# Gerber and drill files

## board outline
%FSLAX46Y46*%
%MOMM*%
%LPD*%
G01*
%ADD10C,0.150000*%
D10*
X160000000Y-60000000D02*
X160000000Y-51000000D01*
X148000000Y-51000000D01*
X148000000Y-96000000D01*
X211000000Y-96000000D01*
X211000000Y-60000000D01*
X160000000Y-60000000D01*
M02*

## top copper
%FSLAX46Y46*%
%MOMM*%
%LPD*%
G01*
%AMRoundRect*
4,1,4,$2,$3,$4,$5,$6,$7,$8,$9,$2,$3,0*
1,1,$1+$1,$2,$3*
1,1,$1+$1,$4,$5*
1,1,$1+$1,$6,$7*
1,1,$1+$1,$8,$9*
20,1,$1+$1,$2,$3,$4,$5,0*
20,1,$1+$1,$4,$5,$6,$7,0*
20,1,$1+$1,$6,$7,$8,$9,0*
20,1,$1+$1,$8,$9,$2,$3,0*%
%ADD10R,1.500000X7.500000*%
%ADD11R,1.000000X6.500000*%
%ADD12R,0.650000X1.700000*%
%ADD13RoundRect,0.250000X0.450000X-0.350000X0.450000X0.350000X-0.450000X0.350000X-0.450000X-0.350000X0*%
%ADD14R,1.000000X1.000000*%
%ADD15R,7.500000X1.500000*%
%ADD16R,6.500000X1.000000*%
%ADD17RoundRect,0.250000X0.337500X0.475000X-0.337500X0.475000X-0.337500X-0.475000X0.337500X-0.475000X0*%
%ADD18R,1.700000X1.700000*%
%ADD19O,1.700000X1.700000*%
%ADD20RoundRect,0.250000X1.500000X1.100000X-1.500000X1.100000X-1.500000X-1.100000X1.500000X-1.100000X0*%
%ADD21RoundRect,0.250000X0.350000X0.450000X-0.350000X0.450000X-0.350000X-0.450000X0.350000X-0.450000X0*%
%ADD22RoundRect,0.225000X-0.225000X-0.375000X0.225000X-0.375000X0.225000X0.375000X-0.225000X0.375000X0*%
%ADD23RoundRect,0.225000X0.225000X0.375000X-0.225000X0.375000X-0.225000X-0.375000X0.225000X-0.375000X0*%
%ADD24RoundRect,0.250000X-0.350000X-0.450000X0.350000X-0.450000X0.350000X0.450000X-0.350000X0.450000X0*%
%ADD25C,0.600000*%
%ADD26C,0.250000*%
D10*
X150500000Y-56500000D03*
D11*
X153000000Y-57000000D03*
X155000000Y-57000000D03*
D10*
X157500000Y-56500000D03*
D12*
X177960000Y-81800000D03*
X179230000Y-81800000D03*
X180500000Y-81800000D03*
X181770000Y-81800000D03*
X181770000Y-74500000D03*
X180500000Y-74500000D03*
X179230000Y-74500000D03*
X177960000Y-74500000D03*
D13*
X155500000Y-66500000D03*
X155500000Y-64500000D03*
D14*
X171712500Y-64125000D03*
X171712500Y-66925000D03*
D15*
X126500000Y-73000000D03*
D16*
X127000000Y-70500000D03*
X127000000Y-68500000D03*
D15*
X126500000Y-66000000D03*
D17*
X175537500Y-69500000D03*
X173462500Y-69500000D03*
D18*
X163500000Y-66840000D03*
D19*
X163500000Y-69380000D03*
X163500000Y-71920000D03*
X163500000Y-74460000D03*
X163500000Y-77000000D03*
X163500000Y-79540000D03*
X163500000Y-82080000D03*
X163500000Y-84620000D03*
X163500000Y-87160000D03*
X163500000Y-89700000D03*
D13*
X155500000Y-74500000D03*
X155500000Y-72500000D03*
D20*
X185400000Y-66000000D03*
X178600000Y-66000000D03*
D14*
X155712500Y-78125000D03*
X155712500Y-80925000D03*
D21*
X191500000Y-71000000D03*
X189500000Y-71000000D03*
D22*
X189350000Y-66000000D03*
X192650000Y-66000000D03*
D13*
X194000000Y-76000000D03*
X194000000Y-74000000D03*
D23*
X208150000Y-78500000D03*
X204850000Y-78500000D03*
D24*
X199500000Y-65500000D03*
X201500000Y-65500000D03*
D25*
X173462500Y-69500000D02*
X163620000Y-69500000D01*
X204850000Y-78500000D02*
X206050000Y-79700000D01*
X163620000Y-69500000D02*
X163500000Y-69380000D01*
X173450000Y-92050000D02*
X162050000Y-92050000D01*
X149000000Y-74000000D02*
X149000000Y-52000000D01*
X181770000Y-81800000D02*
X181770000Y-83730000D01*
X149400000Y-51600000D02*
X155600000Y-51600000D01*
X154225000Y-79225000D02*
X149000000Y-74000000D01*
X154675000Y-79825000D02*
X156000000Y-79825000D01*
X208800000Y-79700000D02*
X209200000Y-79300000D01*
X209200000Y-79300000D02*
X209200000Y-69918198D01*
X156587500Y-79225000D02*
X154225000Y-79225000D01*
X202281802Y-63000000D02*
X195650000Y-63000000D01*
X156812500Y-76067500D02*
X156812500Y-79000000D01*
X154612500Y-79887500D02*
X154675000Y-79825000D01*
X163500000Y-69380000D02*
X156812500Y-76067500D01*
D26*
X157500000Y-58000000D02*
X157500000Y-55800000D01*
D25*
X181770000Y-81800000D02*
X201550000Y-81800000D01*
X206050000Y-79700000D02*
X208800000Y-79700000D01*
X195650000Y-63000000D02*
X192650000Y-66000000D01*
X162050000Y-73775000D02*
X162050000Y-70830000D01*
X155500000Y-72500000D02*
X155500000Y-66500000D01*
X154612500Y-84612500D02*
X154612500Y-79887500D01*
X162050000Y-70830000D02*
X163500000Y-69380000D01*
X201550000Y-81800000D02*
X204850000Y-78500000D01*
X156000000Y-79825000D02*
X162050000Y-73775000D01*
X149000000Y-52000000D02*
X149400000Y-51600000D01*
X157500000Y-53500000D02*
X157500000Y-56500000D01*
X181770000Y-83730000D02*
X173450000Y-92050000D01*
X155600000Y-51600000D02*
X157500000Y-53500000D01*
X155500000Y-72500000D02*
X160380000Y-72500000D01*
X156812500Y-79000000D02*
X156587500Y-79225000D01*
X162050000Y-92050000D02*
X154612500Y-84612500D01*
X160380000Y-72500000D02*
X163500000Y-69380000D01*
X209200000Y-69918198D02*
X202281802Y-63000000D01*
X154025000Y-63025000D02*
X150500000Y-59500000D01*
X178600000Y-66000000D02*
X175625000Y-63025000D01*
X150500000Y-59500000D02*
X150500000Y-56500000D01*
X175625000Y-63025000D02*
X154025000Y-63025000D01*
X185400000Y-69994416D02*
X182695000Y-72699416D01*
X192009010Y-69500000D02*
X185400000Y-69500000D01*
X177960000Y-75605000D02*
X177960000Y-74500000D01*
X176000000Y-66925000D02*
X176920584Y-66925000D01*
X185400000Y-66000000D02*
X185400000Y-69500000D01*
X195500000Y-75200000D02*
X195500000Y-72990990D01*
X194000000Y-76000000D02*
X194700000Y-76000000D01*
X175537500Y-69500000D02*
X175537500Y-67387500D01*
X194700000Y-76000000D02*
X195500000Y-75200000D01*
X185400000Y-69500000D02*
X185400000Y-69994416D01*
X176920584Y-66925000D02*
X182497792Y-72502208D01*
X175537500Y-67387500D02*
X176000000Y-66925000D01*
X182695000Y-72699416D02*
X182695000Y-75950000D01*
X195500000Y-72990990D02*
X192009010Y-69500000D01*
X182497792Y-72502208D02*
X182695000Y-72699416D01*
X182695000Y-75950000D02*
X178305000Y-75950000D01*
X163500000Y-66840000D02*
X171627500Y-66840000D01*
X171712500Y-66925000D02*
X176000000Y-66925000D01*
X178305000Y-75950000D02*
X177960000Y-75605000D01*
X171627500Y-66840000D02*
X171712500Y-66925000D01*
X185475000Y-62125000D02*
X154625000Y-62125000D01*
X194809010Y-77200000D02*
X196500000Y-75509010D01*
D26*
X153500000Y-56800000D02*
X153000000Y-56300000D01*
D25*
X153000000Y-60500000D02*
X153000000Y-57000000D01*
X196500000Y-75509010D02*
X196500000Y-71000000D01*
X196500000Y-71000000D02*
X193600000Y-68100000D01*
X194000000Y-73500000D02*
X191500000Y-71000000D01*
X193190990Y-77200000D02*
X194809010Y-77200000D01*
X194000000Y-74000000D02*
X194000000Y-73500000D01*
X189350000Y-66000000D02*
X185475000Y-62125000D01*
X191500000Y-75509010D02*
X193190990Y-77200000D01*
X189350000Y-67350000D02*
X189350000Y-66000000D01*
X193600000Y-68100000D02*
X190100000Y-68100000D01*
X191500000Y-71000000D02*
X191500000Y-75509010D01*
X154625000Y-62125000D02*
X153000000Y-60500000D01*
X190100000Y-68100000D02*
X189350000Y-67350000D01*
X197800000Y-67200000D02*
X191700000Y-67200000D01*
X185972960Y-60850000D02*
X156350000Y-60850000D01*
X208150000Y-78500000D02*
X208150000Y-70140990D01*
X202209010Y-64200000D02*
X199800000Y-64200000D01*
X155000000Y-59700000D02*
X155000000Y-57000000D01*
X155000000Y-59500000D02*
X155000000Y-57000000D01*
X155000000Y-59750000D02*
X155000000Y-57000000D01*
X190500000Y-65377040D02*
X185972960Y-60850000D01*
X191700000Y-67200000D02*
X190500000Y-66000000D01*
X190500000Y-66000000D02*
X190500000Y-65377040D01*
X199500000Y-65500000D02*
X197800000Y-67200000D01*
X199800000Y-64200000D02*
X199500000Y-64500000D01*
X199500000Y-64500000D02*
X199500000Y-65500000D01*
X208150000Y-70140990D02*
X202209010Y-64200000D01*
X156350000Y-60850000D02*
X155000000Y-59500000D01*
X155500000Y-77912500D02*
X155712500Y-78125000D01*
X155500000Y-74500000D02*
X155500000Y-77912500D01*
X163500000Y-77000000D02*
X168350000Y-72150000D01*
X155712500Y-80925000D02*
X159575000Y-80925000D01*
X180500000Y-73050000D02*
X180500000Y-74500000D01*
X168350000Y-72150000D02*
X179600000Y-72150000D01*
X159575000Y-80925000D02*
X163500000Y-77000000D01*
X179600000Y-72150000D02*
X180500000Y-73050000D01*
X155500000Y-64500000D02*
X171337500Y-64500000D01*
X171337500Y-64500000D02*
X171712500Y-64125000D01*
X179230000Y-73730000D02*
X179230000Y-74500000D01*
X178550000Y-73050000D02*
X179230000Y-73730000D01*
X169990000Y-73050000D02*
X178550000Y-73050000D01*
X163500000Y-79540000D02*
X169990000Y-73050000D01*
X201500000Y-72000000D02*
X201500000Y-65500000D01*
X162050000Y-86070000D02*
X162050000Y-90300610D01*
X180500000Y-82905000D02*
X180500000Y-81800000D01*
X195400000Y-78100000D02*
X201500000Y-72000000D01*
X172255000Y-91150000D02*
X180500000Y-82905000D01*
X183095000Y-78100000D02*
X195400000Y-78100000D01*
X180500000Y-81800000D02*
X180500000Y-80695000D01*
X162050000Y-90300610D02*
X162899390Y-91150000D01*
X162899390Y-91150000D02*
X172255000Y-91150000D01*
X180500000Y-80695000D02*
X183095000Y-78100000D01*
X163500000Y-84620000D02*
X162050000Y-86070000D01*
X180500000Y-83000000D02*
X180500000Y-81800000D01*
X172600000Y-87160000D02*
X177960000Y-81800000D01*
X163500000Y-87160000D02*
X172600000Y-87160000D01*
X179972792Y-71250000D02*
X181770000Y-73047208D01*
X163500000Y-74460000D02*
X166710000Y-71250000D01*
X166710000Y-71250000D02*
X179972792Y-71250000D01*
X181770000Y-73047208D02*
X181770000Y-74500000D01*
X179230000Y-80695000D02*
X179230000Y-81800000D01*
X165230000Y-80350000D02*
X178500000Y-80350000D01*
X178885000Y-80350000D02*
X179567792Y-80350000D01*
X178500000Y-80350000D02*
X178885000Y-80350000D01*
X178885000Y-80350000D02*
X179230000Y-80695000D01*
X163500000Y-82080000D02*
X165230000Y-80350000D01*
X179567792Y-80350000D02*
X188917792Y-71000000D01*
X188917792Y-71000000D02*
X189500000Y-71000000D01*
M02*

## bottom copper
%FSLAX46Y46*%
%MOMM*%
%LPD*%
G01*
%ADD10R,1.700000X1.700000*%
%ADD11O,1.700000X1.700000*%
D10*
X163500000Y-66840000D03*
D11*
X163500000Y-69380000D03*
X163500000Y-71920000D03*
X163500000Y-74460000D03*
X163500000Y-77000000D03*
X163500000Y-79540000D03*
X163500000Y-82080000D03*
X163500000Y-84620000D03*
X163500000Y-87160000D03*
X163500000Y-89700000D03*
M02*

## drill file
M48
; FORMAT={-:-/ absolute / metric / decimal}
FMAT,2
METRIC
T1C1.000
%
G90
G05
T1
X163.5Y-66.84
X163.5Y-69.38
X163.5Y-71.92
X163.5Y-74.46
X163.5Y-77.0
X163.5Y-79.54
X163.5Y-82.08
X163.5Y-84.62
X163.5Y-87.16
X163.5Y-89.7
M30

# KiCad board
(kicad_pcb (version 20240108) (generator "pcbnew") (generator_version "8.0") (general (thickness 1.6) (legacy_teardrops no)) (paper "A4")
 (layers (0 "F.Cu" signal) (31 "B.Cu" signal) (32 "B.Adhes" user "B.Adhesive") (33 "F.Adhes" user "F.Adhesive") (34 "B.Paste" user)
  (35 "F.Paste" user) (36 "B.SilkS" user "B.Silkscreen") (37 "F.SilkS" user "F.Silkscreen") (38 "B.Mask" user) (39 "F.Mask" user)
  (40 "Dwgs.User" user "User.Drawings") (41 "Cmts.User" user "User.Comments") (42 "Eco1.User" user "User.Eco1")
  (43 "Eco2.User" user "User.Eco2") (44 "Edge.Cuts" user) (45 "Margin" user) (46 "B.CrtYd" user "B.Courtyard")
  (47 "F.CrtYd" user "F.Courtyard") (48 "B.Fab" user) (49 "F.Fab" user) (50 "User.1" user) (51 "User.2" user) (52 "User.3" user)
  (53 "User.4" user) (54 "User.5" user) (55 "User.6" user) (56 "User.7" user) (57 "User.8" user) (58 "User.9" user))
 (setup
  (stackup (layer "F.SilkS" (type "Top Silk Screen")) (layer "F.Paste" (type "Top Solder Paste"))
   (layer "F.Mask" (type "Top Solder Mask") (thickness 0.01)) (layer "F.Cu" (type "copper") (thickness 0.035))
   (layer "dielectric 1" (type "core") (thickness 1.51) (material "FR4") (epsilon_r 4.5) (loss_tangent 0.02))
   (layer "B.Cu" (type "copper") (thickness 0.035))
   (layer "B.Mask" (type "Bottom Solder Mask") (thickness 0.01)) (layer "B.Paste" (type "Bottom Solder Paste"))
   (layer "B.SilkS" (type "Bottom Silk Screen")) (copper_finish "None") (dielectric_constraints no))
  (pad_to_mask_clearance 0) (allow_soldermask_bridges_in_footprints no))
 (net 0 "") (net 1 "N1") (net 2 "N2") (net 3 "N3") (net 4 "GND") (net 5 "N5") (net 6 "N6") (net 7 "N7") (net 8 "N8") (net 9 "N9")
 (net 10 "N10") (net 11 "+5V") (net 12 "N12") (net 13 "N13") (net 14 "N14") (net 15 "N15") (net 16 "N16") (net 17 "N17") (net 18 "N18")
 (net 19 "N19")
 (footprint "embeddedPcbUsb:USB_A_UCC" (layer "F.Cu") (at 154 56.7 -90)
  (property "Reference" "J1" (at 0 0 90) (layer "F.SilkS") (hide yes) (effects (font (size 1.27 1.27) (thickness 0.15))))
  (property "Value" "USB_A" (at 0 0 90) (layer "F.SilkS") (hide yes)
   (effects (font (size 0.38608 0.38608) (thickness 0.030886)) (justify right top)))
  (pad "1" smd rect (at -0.2 3.5 270) (size 7.5 1.5) (layers "F.Cu" "F.Paste" "F.Mask") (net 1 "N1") (solder_mask_margin 0.1016))
  (pad "2" smd rect (at 0.3 1 270) (size 6.5 1) (layers "F.Cu" "F.Paste" "F.Mask") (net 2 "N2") (solder_mask_margin 0.1016))
  (pad "3" smd rect (at 0.3 -1 270) (size 6.5 1) (layers "F.Cu" "F.Paste" "F.Mask") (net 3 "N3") (solder_mask_margin 0.1016))
  (pad "4" smd rect (at -0.2 -3.5 270) (size 7.5 1.5) (layers "F.Cu" "F.Paste" "F.Mask") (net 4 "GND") (solder_mask_margin 0.1016)))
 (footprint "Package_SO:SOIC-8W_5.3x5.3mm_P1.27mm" (layer "F.Cu") (at 179.865 78.15 90)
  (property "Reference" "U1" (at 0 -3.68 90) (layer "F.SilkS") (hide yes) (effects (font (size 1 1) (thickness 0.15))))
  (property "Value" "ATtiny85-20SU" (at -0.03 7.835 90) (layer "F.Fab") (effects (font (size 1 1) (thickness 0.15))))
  (pad "1" smd rect (at -3.65 -1.905 90) (size 1.7 0.65) (layers "F.Cu" "F.Paste" "F.Mask") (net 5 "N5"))
  (pad "2" smd rect (at -3.65 -0.635 90) (size 1.7 0.65) (layers "F.Cu" "F.Paste" "F.Mask") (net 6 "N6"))
  (pad "3" smd rect (at -3.65 0.635 90) (size 1.7 0.65) (layers "F.Cu" "F.Paste" "F.Mask") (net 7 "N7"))
  (pad "4" smd rect (at -3.65 1.905 90) (size 1.7 0.65) (layers "F.Cu" "F.Paste" "F.Mask") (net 4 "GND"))
  (pad "5" smd rect (at 3.65 1.905 90) (size 1.7 0.65) (layers "F.Cu" "F.Paste" "F.Mask") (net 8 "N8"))
  (pad "6" smd rect (at 3.65 0.635 90) (size 1.7 0.65) (layers "F.Cu" "F.Paste" "F.Mask") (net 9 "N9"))
  (pad "7" smd rect (at 3.65 -0.635 90) (size 1.7 0.65) (layers "F.Cu" "F.Paste" "F.Mask") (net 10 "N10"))
  (pad "8" smd rect (at 3.65 -1.905 90) (size 1.7 0.65) (layers "F.Cu" "F.Paste" "F.Mask") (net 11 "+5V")))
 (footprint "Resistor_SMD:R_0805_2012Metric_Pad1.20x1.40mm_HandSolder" (layer "F.Cu") (at 155.5 65.5 90)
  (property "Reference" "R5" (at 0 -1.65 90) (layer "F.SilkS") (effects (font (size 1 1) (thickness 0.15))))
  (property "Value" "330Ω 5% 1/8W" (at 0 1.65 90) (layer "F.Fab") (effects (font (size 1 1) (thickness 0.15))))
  (pad "1" smd roundrect (at -1 0 90) (size 1.2 1.4) (layers "F.Cu" "F.Paste" "F.Mask") (roundrect_rratio 0.208333) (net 4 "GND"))
  (pad "2" smd roundrect (at 1 0 90) (size 1.2 1.4) (layers "F.Cu" "F.Paste" "F.Mask") (roundrect_rratio 0.208333) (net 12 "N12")))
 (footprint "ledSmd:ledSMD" (layer "F.Cu") (at 171.7125 65.925 -90)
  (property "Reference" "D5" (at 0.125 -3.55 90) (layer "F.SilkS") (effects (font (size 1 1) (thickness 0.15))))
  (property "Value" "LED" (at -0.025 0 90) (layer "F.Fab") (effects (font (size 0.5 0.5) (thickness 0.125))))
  (pad "1" smd rect (at -1.8 0 270) (size 1 1) (layers "F.Cu" "F.Paste" "F.Mask") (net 12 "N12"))
  (pad "2" smd rect (at 1 0 270) (size 1 1) (layers "F.Cu" "F.Paste" "F.Mask") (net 11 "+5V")))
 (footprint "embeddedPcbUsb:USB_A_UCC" (layer "F.Cu") (at 126.7 69.5)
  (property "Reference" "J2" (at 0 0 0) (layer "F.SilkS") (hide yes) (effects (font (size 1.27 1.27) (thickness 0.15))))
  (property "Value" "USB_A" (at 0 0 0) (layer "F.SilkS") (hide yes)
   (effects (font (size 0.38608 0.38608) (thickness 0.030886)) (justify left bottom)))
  (pad "1" smd rect (at -0.2 3.5) (size 7.5 1.5) (layers "F.Cu" "F.Paste" "F.Mask") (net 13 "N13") (solder_mask_margin 0.1016))
  (pad "2" smd rect (at 0.3 1) (size 6.5 1) (layers "F.Cu" "F.Paste" "F.Mask") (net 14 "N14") (solder_mask_margin 0.1016))
  (pad "3" smd rect (at 0.3 -1) (size 6.5 1) (layers "F.Cu" "F.Paste" "F.Mask") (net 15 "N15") (solder_mask_margin 0.1016))
  (pad "4" smd rect (at -0.2 -3.5) (size 7.5 1.5) (layers "F.Cu" "F.Paste" "F.Mask") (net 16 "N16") (solder_mask_margin 0.1016)))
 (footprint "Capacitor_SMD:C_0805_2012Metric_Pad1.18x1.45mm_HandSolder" (layer "F.Cu") (at 174.5 69.5 180)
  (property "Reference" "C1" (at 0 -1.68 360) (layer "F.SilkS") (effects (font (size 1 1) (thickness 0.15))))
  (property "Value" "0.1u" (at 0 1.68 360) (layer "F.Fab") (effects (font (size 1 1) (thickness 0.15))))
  (pad "1" smd roundrect (at -1.0375 0 180) (size 1.175 1.45) (layers "F.Cu" "F.Paste" "F.Mask") (roundrect_rratio 0.212766) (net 11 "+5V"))
  (pad "2" smd roundrect (at 1.0375 0 180) (size 1.175 1.45) (layers "F.Cu" "F.Paste" "F.Mask") (roundrect_rratio 0.212766) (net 4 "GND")))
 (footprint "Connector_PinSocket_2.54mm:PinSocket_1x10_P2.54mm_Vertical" (layer "F.Cu") (at 163.5 66.84)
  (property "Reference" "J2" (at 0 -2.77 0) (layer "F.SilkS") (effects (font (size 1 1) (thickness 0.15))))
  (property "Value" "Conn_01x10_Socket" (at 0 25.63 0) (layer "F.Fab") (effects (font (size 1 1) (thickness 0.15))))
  (pad "1" thru_hole rect (at 0 0) (size 1.7 1.7) (drill 1) (layers "*.Cu" "*.Mask") (remove_unused_layers no) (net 11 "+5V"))
  (pad "2" thru_hole oval (at 0 2.54) (size 1.7 1.7) (drill 1) (layers "*.Cu" "*.Mask") (remove_unused_layers no) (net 4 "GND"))
  (pad "3" thru_hole oval (at 0 5.08) (size 1.7 1.7) (drill 1) (layers "*.Cu" "*.Mask") (remove_unused_layers no) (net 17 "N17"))
  (pad "4" thru_hole oval (at 0 7.62) (size 1.7 1.7) (drill 1) (layers "*.Cu" "*.Mask") (remove_unused_layers no) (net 8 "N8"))
  (pad "5" thru_hole oval (at 0 10.16) (size 1.7 1.7) (drill 1) (layers "*.Cu" "*.Mask") (remove_unused_layers no) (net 9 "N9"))
  (pad "6" thru_hole oval (at 0 12.7) (size 1.7 1.7) (drill 1) (layers "*.Cu" "*.Mask") (remove_unused_layers no) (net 10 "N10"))
  (pad "7" thru_hole oval (at 0 15.24) (size 1.7 1.7) (drill 1) (layers "*.Cu" "*.Mask") (remove_unused_layers no) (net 6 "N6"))
  (pad "8" thru_hole oval (at 0 17.78) (size 1.7 1.7) (drill 1) (layers "*.Cu" "*.Mask") (remove_unused_layers no) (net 7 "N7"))
  (pad "9" thru_hole oval (at 0 20.32) (size 1.7 1.7) (drill 1) (layers "*.Cu" "*.Mask") (remove_unused_layers no) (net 5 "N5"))
  (pad "10" thru_hole oval (at 0 22.86) (size 1.7 1.7) (drill 1) (layers "*.Cu" "*.Mask") (remove_unused_layers no) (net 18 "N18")))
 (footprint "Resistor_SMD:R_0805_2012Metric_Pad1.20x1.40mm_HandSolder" (layer "F.Cu") (at 155.5 73.5 90)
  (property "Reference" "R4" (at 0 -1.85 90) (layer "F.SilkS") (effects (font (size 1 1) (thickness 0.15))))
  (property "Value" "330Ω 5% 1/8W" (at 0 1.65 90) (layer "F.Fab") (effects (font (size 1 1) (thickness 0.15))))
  (pad "1" smd roundrect (at -1 0 90) (size 1.2 1.4) (layers "F.Cu" "F.Paste" "F.Mask") (roundrect_rratio 0.208333) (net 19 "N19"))
  (pad "2" smd roundrect (at 1 0 90) (size 1.2 1.4) (layers "F.Cu" "F.Paste" "F.Mask") (roundrect_rratio 0.208333) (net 4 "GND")))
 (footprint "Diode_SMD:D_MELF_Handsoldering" (layer "F.Cu") (at 182 66 180)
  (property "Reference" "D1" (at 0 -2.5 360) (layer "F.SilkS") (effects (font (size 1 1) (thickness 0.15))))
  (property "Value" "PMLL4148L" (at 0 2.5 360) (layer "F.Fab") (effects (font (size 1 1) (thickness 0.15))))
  (pad "1" smd roundrect (at -3.4 0 180) (size 3.5 2.7) (layers "F.Cu" "F.Paste" "F.Mask") (roundrect_rratio 0.0925925926) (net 11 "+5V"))
  (pad "2" smd roundrect (at 3.4 0 180) (size 3.5 2.7) (layers "F.Cu" "F.Paste" "F.Mask") (roundrect_rratio 0.0925925926) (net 1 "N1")))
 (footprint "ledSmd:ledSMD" (layer "F.Cu") (at 155.7125 79.925 -90)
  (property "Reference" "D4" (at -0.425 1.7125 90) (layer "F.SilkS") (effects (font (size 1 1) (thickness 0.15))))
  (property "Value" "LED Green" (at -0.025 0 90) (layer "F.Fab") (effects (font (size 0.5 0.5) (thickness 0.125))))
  (pad "1" smd rect (at -1.8 0 270) (size 1 1) (layers "F.Cu" "F.Paste" "F.Mask") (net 19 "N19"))
  (pad "2" smd rect (at 1 0 270) (size 1 1) (layers "F.Cu" "F.Paste" "F.Mask") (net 9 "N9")))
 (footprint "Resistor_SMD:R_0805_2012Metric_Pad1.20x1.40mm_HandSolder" (layer "F.Cu") (at 190.5 71 180)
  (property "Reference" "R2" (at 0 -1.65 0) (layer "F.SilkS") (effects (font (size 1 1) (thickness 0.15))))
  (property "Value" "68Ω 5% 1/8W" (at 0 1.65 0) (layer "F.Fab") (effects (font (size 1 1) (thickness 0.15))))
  (pad "1" smd roundrect (at -1 0 180) (size 1.2 1.4) (layers "F.Cu" "F.Paste" "F.Mask") (roundrect_rratio 0.208333) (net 2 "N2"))
  (pad "2" smd roundrect (at 1 0 180) (size 1.2 1.4) (layers "F.Cu" "F.Paste" "F.Mask") (roundrect_rratio 0.208333) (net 6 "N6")))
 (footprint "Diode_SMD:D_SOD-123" (layer "F.Cu") (at 191 66)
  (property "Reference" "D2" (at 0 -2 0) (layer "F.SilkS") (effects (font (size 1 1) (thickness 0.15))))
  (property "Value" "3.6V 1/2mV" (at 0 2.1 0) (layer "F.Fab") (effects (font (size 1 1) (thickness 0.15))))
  (pad "1" smd roundrect (at -1.65 0) (size 0.9 1.2) (layers "F.Cu" "F.Paste" "F.Mask") (roundrect_rratio 0.25) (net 2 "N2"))
  (pad "2" smd roundrect (at 1.65 0) (size 0.9 1.2) (layers "F.Cu" "F.Paste" "F.Mask") (roundrect_rratio 0.25) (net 4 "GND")))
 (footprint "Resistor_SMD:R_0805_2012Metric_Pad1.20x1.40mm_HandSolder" (layer "F.Cu") (at 194 75 90)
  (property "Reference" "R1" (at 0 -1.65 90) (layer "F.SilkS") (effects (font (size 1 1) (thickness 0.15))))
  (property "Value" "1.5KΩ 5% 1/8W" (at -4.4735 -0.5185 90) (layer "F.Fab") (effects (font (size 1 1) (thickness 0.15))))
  (pad "1" smd roundrect (at -1 0 90) (size 1.2 1.4) (layers "F.Cu" "F.Paste" "F.Mask") (roundrect_rratio 0.208333) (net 11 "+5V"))
  (pad "2" smd roundrect (at 1 0 90) (size 1.2 1.4) (layers "F.Cu" "F.Paste" "F.Mask") (roundrect_rratio 0.208333) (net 2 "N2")))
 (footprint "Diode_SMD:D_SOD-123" (layer "F.Cu") (at 206.5 78.5 180)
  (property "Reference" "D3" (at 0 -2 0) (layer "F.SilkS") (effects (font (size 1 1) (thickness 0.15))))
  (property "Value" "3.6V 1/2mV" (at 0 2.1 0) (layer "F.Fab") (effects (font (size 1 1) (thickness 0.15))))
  (pad "1" smd roundrect (at -1.65 0 180) (size 0.9 1.2) (layers "F.Cu" "F.Paste" "F.Mask") (roundrect_rratio 0.25) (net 3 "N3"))
  (pad "2" smd roundrect (at 1.65 0 180) (size 0.9 1.2) (layers "F.Cu" "F.Paste" "F.Mask") (roundrect_rratio 0.25) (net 4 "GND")))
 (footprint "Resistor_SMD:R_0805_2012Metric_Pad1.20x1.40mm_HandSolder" (layer "F.Cu") (at 200.5 65.5)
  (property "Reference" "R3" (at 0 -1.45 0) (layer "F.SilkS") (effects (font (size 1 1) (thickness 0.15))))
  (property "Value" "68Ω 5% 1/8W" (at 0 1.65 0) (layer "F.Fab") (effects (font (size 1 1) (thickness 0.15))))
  (pad "1" smd roundrect (at -1 0) (size 1.2 1.4) (layers "F.Cu" "F.Paste" "F.Mask") (roundrect_rratio 0.208333) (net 3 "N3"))
  (pad "2" smd roundrect (at 1 0) (size 1.2 1.4) (layers "F.Cu" "F.Paste" "F.Mask") (roundrect_rratio 0.208333) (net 7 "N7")))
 (gr_poly
  (pts (xy 160 60) (xy 160 51) (xy 148 51) (xy 148 96) (xy 211 96) (xy 211 60)) (stroke (width 0.15) (type solid)) (fill none)
  (layer "Edge.Cuts"))
 (segment (start 173.4625 69.5) (end 163.62 69.5) (width 0.6) (layer "F.Cu") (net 4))
 (segment (start 204.85 78.5) (end 206.05 79.7) (width 0.6) (layer "F.Cu") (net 4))
 (segment (start 163.62 69.5) (end 163.5 69.38) (width 0.6) (layer "F.Cu") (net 4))
 (segment (start 173.45 92.05) (end 162.05 92.05) (width 0.6) (layer "F.Cu") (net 4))
 (segment (start 149 74) (end 149 52) (width 0.6) (layer "F.Cu") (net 4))
 (segment (start 181.77 81.8) (end 181.77 83.73) (width 0.6) (layer "F.Cu") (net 4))
 (segment (start 149.4 51.6) (end 155.6 51.6) (width 0.6) (layer "F.Cu") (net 4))
 (segment (start 154.225 79.225) (end 149 74) (width 0.6) (layer "F.Cu") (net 4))
 (segment (start 154.675 79.825) (end 156 79.825) (width 0.6) (layer "F.Cu") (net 4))
 (segment (start 208.8 79.7) (end 209.2 79.3) (width 0.6) (layer "F.Cu") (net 4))
 (segment (start 209.2 79.3) (end 209.2 69.918198) (width 0.6) (layer "F.Cu") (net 4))
 (segment (start 156.5875 79.225) (end 154.225 79.225) (width 0.6) (layer "F.Cu") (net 4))
 (segment (start 202.281802 63) (end 195.65 63) (width 0.6) (layer "F.Cu") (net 4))
 (segment (start 156.8125 76.0675) (end 156.8125 79) (width 0.6) (layer "F.Cu") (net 4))
 (segment (start 154.6125 79.8875) (end 154.675 79.825) (width 0.6) (layer "F.Cu") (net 4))
 (segment (start 163.5 69.38) (end 156.8125 76.0675) (width 0.6) (layer "F.Cu") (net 4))
 (segment (start 157.5 58) (end 157.5 55.8) (width 0.25) (layer "F.Cu") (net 4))
 (segment (start 181.77 81.8) (end 201.55 81.8) (width 0.6) (layer "F.Cu") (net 4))
 (segment (start 206.05 79.7) (end 208.8 79.7) (width 0.6) (layer "F.Cu") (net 4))
 (segment (start 195.65 63) (end 192.65 66) (width 0.6) (layer "F.Cu") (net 4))
 (segment (start 162.05 73.775) (end 162.05 70.83) (width 0.6) (layer "F.Cu") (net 4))
 (segment (start 155.5 72.5) (end 155.5 66.5) (width 0.6) (layer "F.Cu") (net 4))
 (segment (start 154.6125 84.6125) (end 154.6125 79.8875) (width 0.6) (layer "F.Cu") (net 4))
 (segment (start 162.05 70.83) (end 163.5 69.38) (width 0.6) (layer "F.Cu") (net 4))
 (segment (start 201.55 81.8) (end 204.85 78.5) (width 0.6) (layer "F.Cu") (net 4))
 (segment (start 156 79.825) (end 162.05 73.775) (width 0.6) (layer "F.Cu") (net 4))
 (segment (start 149 52) (end 149.4 51.6) (width 0.6) (layer "F.Cu") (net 4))
 (segment (start 157.5 53.5) (end 157.5 56.5) (width 0.6) (layer "F.Cu") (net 4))
 (segment (start 181.77 83.73) (end 173.45 92.05) (width 0.6) (layer "F.Cu") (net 4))
 (segment (start 155.6 51.6) (end 157.5 53.5) (width 0.6) (layer "F.Cu") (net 4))
 (segment (start 155.5 72.5) (end 160.38 72.5) (width 0.6) (layer "F.Cu") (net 4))
 (segment (start 156.8125 79) (end 156.5875 79.225) (width 0.6) (layer "F.Cu") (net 4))
 (segment (start 162.05 92.05) (end 154.6125 84.6125) (width 0.6) (layer "F.Cu") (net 4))
 (segment (start 160.38 72.5) (end 163.5 69.38) (width 0.6) (layer "F.Cu") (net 4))
 (segment (start 209.2 69.918198) (end 202.281802 63) (width 0.6) (layer "F.Cu") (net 4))
 (segment (start 154.025 63.025) (end 150.5 59.5) (width 0.6) (layer "F.Cu") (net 1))
 (segment (start 178.6 66) (end 175.625 63.025) (width 0.6) (layer "F.Cu") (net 1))
 (segment (start 150.5 59.5) (end 150.5 56.5) (width 0.6) (layer "F.Cu") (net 1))
 (segment (start 175.625 63.025) (end 154.025 63.025) (width 0.6) (layer "F.Cu") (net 1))
 (segment (start 185.4 69.994416) (end 182.695 72.699416) (width 0.6) (layer "F.Cu") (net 11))
 (segment (start 192.00901 69.5) (end 185.4 69.5) (width 0.6) (layer "F.Cu") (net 11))
 (segment (start 177.96 75.605) (end 177.96 74.5) (width 0.6) (layer "F.Cu") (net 11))
 (segment (start 176 66.925) (end 176.920584 66.925) (width 0.6) (layer "F.Cu") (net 11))
 (segment (start 185.4 66) (end 185.4 69.5) (width 0.6) (layer "F.Cu") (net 11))
 (segment (start 195.5 75.2) (end 195.5 72.99099) (width 0.6) (layer "F.Cu") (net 11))
 (segment (start 194 76) (end 194.7 76) (width 0.6) (layer "F.Cu") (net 11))
 (segment (start 175.5375 69.5) (end 175.5375 67.3875) (width 0.6) (layer "F.Cu") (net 11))
 (segment (start 194.7 76) (end 195.5 75.2) (width 0.6) (layer "F.Cu") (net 11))
 (segment (start 185.4 69.5) (end 185.4 69.994416) (width 0.6) (layer "F.Cu") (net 11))
 (segment (start 176.920584 66.925) (end 182.497792 72.502208) (width 0.6) (layer "F.Cu") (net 11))
 (segment (start 175.5375 67.3875) (end 176 66.925) (width 0.6) (layer "F.Cu") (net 11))
 (segment (start 182.695 72.699416) (end 182.695 75.95) (width 0.6) (layer "F.Cu") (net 11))
 (segment (start 195.5 72.99099) (end 192.00901 69.5) (width 0.6) (layer "F.Cu") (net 11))
 (segment (start 182.497792 72.502208) (end 182.695 72.699416) (width 0.6) (layer "F.Cu") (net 11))
 (segment (start 182.695 75.95) (end 178.305 75.95) (width 0.6) (layer "F.Cu") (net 11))
 (segment (start 163.5 66.84) (end 171.6275 66.84) (width 0.6) (layer "F.Cu") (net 11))
 (segment (start 171.7125 66.925) (end 176 66.925) (width 0.6) (layer "F.Cu") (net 11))
 (segment (start 178.305 75.95) (end 177.96 75.605) (width 0.6) (layer "F.Cu") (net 11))
 (segment (start 171.6275 66.84) (end 171.7125 66.925) (width 0.6) (layer "F.Cu") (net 11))
 (segment (start 185.475 62.125) (end 154.625 62.125) (width 0.6) (layer "F.Cu") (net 2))
 (segment (start 194.80901 77.2) (end 196.5 75.50901) (width 0.6) (layer "F.Cu") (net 2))
 (segment (start 153.5 56.8) (end 153 56.3) (width 0.25) (layer "F.Cu") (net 2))
 (segment (start 153 60.5) (end 153 57) (width 0.6) (layer "F.Cu") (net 2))
 (segment (start 196.5 75.50901) (end 196.5 71) (width 0.6) (layer "F.Cu") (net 2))
 (segment (start 196.5 71) (end 193.6 68.1) (width 0.6) (layer "F.Cu") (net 2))
 (segment (start 194 73.5) (end 191.5 71) (width 0.6) (layer "F.Cu") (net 2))
 (segment (start 193.19099 77.2) (end 194.80901 77.2) (width 0.6) (layer "F.Cu") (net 2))
 (segment (start 194 74) (end 194 73.5) (width 0.6) (layer "F.Cu") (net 2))
 (segment (start 189.35 66) (end 185.475 62.125) (width 0.6) (layer "F.Cu") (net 2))
 (segment (start 191.5 75.50901) (end 193.19099 77.2) (width 0.6) (layer "F.Cu") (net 2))
 (segment (start 189.35 67.35) (end 189.35 66) (width 0.6) (layer "F.Cu") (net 2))
 (segment (start 193.6 68.1) (end 190.1 68.1) (width 0.6) (layer "F.Cu") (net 2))
 (segment (start 191.5 71) (end 191.5 75.50901) (width 0.6) (layer "F.Cu") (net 2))
 (segment (start 154.625 62.125) (end 153 60.5) (width 0.6) (layer "F.Cu") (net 2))
 (segment (start 190.1 68.1) (end 189.35 67.35) (width 0.6) (layer "F.Cu") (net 2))
 (segment (start 197.8 67.2) (end 191.7 67.2) (width 0.6) (layer "F.Cu") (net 3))
 (segment (start 185.97296 60.85) (end 156.35 60.85) (width 0.6) (layer "F.Cu") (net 3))
 (segment (start 208.15 78.5) (end 208.15 70.14099) (width 0.6) (layer "F.Cu") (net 3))
 (segment (start 202.20901 64.2) (end 199.8 64.2) (width 0.6) (layer "F.Cu") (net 3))
 (segment (start 155 59.7) (end 155 57) (width 0.6) (layer "F.Cu") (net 3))
 (segment (start 155 59.5) (end 155 57) (width 0.6) (layer "F.Cu") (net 3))
 (segment (start 155 59.75) (end 155 57) (width 0.6) (layer "F.Cu") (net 3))
 (segment (start 190.5 65.37704) (end 185.97296 60.85) (width 0.6) (layer "F.Cu") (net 3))
 (segment (start 191.7 67.2) (end 190.5 66) (width 0.6) (layer "F.Cu") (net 3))
 (segment (start 190.5 66) (end 190.5 65.37704) (width 0.6) (layer "F.Cu") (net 3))
 (segment (start 199.5 65.5) (end 197.8 67.2) (width 0.6) (layer "F.Cu") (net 3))
 (segment (start 199.8 64.2) (end 199.5 64.5) (width 0.6) (layer "F.Cu") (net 3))
 (segment (start 199.5 64.5) (end 199.5 65.5) (width 0.6) (layer "F.Cu") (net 3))
 (segment (start 208.15 70.14099) (end 202.20901 64.2) (width 0.6) (layer "F.Cu") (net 3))
 (segment (start 156.35 60.85) (end 155 59.5) (width 0.6) (layer "F.Cu") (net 3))
 (segment (start 155.5 77.9125) (end 155.7125 78.125) (width 0.6) (layer "F.Cu") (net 19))
 (segment (start 155.5 74.5) (end 155.5 77.9125) (width 0.6) (layer "F.Cu") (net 19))
 (segment (start 163.5 77) (end 168.35 72.15) (width 0.6) (layer "F.Cu") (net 9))
 (segment (start 155.7125 80.925) (end 159.575 80.925) (width 0.6) (layer "F.Cu") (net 9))
 (segment (start 180.5 73.05) (end 180.5 74.5) (width 0.6) (layer "F.Cu") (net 9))
 (segment (start 168.35 72.15) (end 179.6 72.15) (width 0.6) (layer "F.Cu") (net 9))
 (segment (start 159.575 80.925) (end 163.5 77) (width 0.6) (layer "F.Cu") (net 9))
 (segment (start 179.6 72.15) (end 180.5 73.05) (width 0.6) (layer "F.Cu") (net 9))
 (segment (start 155.5 64.5) (end 171.3375 64.5) (width 0.6) (layer "F.Cu") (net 12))
 (segment (start 171.3375 64.5) (end 171.7125 64.125) (width 0.6) (layer "F.Cu") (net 12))
 (segment (start 179.23 73.73) (end 179.23 74.5) (width 0.6) (layer "F.Cu") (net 10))
 (segment (start 178.55 73.05) (end 179.23 73.73) (width 0.6) (layer "F.Cu") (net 10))
 (segment (start 169.99 73.05) (end 178.55 73.05) (width 0.6) (layer "F.Cu") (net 10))
 (segment (start 163.5 79.54) (end 169.99 73.05) (width 0.6) (layer "F.Cu") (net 10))
 (segment (start 201.5 72) (end 201.5 65.5) (width 0.6) (layer "F.Cu") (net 7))
 (segment (start 162.05 86.07) (end 162.05 90.30061) (width 0.6) (layer "F.Cu") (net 7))
 (segment (start 180.5 82.905) (end 180.5 81.8) (width 0.6) (layer "F.Cu") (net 7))
 (segment (start 195.4 78.1) (end 201.5 72) (width 0.6) (layer "F.Cu") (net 7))
 (segment (start 172.255 91.15) (end 180.5 82.905) (width 0.6) (layer "F.Cu") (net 7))
 (segment (start 183.095 78.1) (end 195.4 78.1) (width 0.6) (layer "F.Cu") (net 7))
 (segment (start 180.5 81.8) (end 180.5 80.695) (width 0.6) (layer "F.Cu") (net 7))
 (segment (start 162.05 90.30061) (end 162.89939 91.15) (width 0.6) (layer "F.Cu") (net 7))
 (segment (start 162.89939 91.15) (end 172.255 91.15) (width 0.6) (layer "F.Cu") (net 7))
 (segment (start 180.5 80.695) (end 183.095 78.1) (width 0.6) (layer "F.Cu") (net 7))
 (segment (start 163.5 84.62) (end 162.05 86.07) (width 0.6) (layer "F.Cu") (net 7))
 (segment (start 180.5 83) (end 180.5 81.8) (width 0.6) (layer "F.Cu") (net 7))
 (segment (start 172.6 87.16) (end 177.96 81.8) (width 0.6) (layer "F.Cu") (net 5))
 (segment (start 163.5 87.16) (end 172.6 87.16) (width 0.6) (layer "F.Cu") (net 5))
 (segment (start 179.972792 71.25) (end 181.77 73.047208) (width 0.6) (layer "F.Cu") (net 8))
 (segment (start 163.5 74.46) (end 166.71 71.25) (width 0.6) (layer "F.Cu") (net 8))
 (segment (start 166.71 71.25) (end 179.972792 71.25) (width 0.6) (layer "F.Cu") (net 8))
 (segment (start 181.77 73.047208) (end 181.77 74.5) (width 0.6) (layer "F.Cu") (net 8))
 (segment (start 179.23 80.695) (end 179.23 81.8) (width 0.6) (layer "F.Cu") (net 6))
 (segment (start 165.23 80.35) (end 178.5 80.35) (width 0.6) (layer "F.Cu") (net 6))
 (segment (start 178.885 80.35) (end 179.567792 80.35) (width 0.6) (layer "F.Cu") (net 6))
 (segment (start 178.5 80.35) (end 178.885 80.35) (width 0.6) (layer "F.Cu") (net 6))
 (segment (start 178.885 80.35) (end 179.23 80.695) (width 0.6) (layer "F.Cu") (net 6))
 (segment (start 163.5 82.08) (end 165.23 80.35) (width 0.6) (layer "F.Cu") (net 6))
 (segment (start 179.567792 80.35) (end 188.917792 71) (width 0.6) (layer "F.Cu") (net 6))
 (segment (start 188.917792 71) (end 189.5 71) (width 0.6) (layer "F.Cu") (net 6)))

